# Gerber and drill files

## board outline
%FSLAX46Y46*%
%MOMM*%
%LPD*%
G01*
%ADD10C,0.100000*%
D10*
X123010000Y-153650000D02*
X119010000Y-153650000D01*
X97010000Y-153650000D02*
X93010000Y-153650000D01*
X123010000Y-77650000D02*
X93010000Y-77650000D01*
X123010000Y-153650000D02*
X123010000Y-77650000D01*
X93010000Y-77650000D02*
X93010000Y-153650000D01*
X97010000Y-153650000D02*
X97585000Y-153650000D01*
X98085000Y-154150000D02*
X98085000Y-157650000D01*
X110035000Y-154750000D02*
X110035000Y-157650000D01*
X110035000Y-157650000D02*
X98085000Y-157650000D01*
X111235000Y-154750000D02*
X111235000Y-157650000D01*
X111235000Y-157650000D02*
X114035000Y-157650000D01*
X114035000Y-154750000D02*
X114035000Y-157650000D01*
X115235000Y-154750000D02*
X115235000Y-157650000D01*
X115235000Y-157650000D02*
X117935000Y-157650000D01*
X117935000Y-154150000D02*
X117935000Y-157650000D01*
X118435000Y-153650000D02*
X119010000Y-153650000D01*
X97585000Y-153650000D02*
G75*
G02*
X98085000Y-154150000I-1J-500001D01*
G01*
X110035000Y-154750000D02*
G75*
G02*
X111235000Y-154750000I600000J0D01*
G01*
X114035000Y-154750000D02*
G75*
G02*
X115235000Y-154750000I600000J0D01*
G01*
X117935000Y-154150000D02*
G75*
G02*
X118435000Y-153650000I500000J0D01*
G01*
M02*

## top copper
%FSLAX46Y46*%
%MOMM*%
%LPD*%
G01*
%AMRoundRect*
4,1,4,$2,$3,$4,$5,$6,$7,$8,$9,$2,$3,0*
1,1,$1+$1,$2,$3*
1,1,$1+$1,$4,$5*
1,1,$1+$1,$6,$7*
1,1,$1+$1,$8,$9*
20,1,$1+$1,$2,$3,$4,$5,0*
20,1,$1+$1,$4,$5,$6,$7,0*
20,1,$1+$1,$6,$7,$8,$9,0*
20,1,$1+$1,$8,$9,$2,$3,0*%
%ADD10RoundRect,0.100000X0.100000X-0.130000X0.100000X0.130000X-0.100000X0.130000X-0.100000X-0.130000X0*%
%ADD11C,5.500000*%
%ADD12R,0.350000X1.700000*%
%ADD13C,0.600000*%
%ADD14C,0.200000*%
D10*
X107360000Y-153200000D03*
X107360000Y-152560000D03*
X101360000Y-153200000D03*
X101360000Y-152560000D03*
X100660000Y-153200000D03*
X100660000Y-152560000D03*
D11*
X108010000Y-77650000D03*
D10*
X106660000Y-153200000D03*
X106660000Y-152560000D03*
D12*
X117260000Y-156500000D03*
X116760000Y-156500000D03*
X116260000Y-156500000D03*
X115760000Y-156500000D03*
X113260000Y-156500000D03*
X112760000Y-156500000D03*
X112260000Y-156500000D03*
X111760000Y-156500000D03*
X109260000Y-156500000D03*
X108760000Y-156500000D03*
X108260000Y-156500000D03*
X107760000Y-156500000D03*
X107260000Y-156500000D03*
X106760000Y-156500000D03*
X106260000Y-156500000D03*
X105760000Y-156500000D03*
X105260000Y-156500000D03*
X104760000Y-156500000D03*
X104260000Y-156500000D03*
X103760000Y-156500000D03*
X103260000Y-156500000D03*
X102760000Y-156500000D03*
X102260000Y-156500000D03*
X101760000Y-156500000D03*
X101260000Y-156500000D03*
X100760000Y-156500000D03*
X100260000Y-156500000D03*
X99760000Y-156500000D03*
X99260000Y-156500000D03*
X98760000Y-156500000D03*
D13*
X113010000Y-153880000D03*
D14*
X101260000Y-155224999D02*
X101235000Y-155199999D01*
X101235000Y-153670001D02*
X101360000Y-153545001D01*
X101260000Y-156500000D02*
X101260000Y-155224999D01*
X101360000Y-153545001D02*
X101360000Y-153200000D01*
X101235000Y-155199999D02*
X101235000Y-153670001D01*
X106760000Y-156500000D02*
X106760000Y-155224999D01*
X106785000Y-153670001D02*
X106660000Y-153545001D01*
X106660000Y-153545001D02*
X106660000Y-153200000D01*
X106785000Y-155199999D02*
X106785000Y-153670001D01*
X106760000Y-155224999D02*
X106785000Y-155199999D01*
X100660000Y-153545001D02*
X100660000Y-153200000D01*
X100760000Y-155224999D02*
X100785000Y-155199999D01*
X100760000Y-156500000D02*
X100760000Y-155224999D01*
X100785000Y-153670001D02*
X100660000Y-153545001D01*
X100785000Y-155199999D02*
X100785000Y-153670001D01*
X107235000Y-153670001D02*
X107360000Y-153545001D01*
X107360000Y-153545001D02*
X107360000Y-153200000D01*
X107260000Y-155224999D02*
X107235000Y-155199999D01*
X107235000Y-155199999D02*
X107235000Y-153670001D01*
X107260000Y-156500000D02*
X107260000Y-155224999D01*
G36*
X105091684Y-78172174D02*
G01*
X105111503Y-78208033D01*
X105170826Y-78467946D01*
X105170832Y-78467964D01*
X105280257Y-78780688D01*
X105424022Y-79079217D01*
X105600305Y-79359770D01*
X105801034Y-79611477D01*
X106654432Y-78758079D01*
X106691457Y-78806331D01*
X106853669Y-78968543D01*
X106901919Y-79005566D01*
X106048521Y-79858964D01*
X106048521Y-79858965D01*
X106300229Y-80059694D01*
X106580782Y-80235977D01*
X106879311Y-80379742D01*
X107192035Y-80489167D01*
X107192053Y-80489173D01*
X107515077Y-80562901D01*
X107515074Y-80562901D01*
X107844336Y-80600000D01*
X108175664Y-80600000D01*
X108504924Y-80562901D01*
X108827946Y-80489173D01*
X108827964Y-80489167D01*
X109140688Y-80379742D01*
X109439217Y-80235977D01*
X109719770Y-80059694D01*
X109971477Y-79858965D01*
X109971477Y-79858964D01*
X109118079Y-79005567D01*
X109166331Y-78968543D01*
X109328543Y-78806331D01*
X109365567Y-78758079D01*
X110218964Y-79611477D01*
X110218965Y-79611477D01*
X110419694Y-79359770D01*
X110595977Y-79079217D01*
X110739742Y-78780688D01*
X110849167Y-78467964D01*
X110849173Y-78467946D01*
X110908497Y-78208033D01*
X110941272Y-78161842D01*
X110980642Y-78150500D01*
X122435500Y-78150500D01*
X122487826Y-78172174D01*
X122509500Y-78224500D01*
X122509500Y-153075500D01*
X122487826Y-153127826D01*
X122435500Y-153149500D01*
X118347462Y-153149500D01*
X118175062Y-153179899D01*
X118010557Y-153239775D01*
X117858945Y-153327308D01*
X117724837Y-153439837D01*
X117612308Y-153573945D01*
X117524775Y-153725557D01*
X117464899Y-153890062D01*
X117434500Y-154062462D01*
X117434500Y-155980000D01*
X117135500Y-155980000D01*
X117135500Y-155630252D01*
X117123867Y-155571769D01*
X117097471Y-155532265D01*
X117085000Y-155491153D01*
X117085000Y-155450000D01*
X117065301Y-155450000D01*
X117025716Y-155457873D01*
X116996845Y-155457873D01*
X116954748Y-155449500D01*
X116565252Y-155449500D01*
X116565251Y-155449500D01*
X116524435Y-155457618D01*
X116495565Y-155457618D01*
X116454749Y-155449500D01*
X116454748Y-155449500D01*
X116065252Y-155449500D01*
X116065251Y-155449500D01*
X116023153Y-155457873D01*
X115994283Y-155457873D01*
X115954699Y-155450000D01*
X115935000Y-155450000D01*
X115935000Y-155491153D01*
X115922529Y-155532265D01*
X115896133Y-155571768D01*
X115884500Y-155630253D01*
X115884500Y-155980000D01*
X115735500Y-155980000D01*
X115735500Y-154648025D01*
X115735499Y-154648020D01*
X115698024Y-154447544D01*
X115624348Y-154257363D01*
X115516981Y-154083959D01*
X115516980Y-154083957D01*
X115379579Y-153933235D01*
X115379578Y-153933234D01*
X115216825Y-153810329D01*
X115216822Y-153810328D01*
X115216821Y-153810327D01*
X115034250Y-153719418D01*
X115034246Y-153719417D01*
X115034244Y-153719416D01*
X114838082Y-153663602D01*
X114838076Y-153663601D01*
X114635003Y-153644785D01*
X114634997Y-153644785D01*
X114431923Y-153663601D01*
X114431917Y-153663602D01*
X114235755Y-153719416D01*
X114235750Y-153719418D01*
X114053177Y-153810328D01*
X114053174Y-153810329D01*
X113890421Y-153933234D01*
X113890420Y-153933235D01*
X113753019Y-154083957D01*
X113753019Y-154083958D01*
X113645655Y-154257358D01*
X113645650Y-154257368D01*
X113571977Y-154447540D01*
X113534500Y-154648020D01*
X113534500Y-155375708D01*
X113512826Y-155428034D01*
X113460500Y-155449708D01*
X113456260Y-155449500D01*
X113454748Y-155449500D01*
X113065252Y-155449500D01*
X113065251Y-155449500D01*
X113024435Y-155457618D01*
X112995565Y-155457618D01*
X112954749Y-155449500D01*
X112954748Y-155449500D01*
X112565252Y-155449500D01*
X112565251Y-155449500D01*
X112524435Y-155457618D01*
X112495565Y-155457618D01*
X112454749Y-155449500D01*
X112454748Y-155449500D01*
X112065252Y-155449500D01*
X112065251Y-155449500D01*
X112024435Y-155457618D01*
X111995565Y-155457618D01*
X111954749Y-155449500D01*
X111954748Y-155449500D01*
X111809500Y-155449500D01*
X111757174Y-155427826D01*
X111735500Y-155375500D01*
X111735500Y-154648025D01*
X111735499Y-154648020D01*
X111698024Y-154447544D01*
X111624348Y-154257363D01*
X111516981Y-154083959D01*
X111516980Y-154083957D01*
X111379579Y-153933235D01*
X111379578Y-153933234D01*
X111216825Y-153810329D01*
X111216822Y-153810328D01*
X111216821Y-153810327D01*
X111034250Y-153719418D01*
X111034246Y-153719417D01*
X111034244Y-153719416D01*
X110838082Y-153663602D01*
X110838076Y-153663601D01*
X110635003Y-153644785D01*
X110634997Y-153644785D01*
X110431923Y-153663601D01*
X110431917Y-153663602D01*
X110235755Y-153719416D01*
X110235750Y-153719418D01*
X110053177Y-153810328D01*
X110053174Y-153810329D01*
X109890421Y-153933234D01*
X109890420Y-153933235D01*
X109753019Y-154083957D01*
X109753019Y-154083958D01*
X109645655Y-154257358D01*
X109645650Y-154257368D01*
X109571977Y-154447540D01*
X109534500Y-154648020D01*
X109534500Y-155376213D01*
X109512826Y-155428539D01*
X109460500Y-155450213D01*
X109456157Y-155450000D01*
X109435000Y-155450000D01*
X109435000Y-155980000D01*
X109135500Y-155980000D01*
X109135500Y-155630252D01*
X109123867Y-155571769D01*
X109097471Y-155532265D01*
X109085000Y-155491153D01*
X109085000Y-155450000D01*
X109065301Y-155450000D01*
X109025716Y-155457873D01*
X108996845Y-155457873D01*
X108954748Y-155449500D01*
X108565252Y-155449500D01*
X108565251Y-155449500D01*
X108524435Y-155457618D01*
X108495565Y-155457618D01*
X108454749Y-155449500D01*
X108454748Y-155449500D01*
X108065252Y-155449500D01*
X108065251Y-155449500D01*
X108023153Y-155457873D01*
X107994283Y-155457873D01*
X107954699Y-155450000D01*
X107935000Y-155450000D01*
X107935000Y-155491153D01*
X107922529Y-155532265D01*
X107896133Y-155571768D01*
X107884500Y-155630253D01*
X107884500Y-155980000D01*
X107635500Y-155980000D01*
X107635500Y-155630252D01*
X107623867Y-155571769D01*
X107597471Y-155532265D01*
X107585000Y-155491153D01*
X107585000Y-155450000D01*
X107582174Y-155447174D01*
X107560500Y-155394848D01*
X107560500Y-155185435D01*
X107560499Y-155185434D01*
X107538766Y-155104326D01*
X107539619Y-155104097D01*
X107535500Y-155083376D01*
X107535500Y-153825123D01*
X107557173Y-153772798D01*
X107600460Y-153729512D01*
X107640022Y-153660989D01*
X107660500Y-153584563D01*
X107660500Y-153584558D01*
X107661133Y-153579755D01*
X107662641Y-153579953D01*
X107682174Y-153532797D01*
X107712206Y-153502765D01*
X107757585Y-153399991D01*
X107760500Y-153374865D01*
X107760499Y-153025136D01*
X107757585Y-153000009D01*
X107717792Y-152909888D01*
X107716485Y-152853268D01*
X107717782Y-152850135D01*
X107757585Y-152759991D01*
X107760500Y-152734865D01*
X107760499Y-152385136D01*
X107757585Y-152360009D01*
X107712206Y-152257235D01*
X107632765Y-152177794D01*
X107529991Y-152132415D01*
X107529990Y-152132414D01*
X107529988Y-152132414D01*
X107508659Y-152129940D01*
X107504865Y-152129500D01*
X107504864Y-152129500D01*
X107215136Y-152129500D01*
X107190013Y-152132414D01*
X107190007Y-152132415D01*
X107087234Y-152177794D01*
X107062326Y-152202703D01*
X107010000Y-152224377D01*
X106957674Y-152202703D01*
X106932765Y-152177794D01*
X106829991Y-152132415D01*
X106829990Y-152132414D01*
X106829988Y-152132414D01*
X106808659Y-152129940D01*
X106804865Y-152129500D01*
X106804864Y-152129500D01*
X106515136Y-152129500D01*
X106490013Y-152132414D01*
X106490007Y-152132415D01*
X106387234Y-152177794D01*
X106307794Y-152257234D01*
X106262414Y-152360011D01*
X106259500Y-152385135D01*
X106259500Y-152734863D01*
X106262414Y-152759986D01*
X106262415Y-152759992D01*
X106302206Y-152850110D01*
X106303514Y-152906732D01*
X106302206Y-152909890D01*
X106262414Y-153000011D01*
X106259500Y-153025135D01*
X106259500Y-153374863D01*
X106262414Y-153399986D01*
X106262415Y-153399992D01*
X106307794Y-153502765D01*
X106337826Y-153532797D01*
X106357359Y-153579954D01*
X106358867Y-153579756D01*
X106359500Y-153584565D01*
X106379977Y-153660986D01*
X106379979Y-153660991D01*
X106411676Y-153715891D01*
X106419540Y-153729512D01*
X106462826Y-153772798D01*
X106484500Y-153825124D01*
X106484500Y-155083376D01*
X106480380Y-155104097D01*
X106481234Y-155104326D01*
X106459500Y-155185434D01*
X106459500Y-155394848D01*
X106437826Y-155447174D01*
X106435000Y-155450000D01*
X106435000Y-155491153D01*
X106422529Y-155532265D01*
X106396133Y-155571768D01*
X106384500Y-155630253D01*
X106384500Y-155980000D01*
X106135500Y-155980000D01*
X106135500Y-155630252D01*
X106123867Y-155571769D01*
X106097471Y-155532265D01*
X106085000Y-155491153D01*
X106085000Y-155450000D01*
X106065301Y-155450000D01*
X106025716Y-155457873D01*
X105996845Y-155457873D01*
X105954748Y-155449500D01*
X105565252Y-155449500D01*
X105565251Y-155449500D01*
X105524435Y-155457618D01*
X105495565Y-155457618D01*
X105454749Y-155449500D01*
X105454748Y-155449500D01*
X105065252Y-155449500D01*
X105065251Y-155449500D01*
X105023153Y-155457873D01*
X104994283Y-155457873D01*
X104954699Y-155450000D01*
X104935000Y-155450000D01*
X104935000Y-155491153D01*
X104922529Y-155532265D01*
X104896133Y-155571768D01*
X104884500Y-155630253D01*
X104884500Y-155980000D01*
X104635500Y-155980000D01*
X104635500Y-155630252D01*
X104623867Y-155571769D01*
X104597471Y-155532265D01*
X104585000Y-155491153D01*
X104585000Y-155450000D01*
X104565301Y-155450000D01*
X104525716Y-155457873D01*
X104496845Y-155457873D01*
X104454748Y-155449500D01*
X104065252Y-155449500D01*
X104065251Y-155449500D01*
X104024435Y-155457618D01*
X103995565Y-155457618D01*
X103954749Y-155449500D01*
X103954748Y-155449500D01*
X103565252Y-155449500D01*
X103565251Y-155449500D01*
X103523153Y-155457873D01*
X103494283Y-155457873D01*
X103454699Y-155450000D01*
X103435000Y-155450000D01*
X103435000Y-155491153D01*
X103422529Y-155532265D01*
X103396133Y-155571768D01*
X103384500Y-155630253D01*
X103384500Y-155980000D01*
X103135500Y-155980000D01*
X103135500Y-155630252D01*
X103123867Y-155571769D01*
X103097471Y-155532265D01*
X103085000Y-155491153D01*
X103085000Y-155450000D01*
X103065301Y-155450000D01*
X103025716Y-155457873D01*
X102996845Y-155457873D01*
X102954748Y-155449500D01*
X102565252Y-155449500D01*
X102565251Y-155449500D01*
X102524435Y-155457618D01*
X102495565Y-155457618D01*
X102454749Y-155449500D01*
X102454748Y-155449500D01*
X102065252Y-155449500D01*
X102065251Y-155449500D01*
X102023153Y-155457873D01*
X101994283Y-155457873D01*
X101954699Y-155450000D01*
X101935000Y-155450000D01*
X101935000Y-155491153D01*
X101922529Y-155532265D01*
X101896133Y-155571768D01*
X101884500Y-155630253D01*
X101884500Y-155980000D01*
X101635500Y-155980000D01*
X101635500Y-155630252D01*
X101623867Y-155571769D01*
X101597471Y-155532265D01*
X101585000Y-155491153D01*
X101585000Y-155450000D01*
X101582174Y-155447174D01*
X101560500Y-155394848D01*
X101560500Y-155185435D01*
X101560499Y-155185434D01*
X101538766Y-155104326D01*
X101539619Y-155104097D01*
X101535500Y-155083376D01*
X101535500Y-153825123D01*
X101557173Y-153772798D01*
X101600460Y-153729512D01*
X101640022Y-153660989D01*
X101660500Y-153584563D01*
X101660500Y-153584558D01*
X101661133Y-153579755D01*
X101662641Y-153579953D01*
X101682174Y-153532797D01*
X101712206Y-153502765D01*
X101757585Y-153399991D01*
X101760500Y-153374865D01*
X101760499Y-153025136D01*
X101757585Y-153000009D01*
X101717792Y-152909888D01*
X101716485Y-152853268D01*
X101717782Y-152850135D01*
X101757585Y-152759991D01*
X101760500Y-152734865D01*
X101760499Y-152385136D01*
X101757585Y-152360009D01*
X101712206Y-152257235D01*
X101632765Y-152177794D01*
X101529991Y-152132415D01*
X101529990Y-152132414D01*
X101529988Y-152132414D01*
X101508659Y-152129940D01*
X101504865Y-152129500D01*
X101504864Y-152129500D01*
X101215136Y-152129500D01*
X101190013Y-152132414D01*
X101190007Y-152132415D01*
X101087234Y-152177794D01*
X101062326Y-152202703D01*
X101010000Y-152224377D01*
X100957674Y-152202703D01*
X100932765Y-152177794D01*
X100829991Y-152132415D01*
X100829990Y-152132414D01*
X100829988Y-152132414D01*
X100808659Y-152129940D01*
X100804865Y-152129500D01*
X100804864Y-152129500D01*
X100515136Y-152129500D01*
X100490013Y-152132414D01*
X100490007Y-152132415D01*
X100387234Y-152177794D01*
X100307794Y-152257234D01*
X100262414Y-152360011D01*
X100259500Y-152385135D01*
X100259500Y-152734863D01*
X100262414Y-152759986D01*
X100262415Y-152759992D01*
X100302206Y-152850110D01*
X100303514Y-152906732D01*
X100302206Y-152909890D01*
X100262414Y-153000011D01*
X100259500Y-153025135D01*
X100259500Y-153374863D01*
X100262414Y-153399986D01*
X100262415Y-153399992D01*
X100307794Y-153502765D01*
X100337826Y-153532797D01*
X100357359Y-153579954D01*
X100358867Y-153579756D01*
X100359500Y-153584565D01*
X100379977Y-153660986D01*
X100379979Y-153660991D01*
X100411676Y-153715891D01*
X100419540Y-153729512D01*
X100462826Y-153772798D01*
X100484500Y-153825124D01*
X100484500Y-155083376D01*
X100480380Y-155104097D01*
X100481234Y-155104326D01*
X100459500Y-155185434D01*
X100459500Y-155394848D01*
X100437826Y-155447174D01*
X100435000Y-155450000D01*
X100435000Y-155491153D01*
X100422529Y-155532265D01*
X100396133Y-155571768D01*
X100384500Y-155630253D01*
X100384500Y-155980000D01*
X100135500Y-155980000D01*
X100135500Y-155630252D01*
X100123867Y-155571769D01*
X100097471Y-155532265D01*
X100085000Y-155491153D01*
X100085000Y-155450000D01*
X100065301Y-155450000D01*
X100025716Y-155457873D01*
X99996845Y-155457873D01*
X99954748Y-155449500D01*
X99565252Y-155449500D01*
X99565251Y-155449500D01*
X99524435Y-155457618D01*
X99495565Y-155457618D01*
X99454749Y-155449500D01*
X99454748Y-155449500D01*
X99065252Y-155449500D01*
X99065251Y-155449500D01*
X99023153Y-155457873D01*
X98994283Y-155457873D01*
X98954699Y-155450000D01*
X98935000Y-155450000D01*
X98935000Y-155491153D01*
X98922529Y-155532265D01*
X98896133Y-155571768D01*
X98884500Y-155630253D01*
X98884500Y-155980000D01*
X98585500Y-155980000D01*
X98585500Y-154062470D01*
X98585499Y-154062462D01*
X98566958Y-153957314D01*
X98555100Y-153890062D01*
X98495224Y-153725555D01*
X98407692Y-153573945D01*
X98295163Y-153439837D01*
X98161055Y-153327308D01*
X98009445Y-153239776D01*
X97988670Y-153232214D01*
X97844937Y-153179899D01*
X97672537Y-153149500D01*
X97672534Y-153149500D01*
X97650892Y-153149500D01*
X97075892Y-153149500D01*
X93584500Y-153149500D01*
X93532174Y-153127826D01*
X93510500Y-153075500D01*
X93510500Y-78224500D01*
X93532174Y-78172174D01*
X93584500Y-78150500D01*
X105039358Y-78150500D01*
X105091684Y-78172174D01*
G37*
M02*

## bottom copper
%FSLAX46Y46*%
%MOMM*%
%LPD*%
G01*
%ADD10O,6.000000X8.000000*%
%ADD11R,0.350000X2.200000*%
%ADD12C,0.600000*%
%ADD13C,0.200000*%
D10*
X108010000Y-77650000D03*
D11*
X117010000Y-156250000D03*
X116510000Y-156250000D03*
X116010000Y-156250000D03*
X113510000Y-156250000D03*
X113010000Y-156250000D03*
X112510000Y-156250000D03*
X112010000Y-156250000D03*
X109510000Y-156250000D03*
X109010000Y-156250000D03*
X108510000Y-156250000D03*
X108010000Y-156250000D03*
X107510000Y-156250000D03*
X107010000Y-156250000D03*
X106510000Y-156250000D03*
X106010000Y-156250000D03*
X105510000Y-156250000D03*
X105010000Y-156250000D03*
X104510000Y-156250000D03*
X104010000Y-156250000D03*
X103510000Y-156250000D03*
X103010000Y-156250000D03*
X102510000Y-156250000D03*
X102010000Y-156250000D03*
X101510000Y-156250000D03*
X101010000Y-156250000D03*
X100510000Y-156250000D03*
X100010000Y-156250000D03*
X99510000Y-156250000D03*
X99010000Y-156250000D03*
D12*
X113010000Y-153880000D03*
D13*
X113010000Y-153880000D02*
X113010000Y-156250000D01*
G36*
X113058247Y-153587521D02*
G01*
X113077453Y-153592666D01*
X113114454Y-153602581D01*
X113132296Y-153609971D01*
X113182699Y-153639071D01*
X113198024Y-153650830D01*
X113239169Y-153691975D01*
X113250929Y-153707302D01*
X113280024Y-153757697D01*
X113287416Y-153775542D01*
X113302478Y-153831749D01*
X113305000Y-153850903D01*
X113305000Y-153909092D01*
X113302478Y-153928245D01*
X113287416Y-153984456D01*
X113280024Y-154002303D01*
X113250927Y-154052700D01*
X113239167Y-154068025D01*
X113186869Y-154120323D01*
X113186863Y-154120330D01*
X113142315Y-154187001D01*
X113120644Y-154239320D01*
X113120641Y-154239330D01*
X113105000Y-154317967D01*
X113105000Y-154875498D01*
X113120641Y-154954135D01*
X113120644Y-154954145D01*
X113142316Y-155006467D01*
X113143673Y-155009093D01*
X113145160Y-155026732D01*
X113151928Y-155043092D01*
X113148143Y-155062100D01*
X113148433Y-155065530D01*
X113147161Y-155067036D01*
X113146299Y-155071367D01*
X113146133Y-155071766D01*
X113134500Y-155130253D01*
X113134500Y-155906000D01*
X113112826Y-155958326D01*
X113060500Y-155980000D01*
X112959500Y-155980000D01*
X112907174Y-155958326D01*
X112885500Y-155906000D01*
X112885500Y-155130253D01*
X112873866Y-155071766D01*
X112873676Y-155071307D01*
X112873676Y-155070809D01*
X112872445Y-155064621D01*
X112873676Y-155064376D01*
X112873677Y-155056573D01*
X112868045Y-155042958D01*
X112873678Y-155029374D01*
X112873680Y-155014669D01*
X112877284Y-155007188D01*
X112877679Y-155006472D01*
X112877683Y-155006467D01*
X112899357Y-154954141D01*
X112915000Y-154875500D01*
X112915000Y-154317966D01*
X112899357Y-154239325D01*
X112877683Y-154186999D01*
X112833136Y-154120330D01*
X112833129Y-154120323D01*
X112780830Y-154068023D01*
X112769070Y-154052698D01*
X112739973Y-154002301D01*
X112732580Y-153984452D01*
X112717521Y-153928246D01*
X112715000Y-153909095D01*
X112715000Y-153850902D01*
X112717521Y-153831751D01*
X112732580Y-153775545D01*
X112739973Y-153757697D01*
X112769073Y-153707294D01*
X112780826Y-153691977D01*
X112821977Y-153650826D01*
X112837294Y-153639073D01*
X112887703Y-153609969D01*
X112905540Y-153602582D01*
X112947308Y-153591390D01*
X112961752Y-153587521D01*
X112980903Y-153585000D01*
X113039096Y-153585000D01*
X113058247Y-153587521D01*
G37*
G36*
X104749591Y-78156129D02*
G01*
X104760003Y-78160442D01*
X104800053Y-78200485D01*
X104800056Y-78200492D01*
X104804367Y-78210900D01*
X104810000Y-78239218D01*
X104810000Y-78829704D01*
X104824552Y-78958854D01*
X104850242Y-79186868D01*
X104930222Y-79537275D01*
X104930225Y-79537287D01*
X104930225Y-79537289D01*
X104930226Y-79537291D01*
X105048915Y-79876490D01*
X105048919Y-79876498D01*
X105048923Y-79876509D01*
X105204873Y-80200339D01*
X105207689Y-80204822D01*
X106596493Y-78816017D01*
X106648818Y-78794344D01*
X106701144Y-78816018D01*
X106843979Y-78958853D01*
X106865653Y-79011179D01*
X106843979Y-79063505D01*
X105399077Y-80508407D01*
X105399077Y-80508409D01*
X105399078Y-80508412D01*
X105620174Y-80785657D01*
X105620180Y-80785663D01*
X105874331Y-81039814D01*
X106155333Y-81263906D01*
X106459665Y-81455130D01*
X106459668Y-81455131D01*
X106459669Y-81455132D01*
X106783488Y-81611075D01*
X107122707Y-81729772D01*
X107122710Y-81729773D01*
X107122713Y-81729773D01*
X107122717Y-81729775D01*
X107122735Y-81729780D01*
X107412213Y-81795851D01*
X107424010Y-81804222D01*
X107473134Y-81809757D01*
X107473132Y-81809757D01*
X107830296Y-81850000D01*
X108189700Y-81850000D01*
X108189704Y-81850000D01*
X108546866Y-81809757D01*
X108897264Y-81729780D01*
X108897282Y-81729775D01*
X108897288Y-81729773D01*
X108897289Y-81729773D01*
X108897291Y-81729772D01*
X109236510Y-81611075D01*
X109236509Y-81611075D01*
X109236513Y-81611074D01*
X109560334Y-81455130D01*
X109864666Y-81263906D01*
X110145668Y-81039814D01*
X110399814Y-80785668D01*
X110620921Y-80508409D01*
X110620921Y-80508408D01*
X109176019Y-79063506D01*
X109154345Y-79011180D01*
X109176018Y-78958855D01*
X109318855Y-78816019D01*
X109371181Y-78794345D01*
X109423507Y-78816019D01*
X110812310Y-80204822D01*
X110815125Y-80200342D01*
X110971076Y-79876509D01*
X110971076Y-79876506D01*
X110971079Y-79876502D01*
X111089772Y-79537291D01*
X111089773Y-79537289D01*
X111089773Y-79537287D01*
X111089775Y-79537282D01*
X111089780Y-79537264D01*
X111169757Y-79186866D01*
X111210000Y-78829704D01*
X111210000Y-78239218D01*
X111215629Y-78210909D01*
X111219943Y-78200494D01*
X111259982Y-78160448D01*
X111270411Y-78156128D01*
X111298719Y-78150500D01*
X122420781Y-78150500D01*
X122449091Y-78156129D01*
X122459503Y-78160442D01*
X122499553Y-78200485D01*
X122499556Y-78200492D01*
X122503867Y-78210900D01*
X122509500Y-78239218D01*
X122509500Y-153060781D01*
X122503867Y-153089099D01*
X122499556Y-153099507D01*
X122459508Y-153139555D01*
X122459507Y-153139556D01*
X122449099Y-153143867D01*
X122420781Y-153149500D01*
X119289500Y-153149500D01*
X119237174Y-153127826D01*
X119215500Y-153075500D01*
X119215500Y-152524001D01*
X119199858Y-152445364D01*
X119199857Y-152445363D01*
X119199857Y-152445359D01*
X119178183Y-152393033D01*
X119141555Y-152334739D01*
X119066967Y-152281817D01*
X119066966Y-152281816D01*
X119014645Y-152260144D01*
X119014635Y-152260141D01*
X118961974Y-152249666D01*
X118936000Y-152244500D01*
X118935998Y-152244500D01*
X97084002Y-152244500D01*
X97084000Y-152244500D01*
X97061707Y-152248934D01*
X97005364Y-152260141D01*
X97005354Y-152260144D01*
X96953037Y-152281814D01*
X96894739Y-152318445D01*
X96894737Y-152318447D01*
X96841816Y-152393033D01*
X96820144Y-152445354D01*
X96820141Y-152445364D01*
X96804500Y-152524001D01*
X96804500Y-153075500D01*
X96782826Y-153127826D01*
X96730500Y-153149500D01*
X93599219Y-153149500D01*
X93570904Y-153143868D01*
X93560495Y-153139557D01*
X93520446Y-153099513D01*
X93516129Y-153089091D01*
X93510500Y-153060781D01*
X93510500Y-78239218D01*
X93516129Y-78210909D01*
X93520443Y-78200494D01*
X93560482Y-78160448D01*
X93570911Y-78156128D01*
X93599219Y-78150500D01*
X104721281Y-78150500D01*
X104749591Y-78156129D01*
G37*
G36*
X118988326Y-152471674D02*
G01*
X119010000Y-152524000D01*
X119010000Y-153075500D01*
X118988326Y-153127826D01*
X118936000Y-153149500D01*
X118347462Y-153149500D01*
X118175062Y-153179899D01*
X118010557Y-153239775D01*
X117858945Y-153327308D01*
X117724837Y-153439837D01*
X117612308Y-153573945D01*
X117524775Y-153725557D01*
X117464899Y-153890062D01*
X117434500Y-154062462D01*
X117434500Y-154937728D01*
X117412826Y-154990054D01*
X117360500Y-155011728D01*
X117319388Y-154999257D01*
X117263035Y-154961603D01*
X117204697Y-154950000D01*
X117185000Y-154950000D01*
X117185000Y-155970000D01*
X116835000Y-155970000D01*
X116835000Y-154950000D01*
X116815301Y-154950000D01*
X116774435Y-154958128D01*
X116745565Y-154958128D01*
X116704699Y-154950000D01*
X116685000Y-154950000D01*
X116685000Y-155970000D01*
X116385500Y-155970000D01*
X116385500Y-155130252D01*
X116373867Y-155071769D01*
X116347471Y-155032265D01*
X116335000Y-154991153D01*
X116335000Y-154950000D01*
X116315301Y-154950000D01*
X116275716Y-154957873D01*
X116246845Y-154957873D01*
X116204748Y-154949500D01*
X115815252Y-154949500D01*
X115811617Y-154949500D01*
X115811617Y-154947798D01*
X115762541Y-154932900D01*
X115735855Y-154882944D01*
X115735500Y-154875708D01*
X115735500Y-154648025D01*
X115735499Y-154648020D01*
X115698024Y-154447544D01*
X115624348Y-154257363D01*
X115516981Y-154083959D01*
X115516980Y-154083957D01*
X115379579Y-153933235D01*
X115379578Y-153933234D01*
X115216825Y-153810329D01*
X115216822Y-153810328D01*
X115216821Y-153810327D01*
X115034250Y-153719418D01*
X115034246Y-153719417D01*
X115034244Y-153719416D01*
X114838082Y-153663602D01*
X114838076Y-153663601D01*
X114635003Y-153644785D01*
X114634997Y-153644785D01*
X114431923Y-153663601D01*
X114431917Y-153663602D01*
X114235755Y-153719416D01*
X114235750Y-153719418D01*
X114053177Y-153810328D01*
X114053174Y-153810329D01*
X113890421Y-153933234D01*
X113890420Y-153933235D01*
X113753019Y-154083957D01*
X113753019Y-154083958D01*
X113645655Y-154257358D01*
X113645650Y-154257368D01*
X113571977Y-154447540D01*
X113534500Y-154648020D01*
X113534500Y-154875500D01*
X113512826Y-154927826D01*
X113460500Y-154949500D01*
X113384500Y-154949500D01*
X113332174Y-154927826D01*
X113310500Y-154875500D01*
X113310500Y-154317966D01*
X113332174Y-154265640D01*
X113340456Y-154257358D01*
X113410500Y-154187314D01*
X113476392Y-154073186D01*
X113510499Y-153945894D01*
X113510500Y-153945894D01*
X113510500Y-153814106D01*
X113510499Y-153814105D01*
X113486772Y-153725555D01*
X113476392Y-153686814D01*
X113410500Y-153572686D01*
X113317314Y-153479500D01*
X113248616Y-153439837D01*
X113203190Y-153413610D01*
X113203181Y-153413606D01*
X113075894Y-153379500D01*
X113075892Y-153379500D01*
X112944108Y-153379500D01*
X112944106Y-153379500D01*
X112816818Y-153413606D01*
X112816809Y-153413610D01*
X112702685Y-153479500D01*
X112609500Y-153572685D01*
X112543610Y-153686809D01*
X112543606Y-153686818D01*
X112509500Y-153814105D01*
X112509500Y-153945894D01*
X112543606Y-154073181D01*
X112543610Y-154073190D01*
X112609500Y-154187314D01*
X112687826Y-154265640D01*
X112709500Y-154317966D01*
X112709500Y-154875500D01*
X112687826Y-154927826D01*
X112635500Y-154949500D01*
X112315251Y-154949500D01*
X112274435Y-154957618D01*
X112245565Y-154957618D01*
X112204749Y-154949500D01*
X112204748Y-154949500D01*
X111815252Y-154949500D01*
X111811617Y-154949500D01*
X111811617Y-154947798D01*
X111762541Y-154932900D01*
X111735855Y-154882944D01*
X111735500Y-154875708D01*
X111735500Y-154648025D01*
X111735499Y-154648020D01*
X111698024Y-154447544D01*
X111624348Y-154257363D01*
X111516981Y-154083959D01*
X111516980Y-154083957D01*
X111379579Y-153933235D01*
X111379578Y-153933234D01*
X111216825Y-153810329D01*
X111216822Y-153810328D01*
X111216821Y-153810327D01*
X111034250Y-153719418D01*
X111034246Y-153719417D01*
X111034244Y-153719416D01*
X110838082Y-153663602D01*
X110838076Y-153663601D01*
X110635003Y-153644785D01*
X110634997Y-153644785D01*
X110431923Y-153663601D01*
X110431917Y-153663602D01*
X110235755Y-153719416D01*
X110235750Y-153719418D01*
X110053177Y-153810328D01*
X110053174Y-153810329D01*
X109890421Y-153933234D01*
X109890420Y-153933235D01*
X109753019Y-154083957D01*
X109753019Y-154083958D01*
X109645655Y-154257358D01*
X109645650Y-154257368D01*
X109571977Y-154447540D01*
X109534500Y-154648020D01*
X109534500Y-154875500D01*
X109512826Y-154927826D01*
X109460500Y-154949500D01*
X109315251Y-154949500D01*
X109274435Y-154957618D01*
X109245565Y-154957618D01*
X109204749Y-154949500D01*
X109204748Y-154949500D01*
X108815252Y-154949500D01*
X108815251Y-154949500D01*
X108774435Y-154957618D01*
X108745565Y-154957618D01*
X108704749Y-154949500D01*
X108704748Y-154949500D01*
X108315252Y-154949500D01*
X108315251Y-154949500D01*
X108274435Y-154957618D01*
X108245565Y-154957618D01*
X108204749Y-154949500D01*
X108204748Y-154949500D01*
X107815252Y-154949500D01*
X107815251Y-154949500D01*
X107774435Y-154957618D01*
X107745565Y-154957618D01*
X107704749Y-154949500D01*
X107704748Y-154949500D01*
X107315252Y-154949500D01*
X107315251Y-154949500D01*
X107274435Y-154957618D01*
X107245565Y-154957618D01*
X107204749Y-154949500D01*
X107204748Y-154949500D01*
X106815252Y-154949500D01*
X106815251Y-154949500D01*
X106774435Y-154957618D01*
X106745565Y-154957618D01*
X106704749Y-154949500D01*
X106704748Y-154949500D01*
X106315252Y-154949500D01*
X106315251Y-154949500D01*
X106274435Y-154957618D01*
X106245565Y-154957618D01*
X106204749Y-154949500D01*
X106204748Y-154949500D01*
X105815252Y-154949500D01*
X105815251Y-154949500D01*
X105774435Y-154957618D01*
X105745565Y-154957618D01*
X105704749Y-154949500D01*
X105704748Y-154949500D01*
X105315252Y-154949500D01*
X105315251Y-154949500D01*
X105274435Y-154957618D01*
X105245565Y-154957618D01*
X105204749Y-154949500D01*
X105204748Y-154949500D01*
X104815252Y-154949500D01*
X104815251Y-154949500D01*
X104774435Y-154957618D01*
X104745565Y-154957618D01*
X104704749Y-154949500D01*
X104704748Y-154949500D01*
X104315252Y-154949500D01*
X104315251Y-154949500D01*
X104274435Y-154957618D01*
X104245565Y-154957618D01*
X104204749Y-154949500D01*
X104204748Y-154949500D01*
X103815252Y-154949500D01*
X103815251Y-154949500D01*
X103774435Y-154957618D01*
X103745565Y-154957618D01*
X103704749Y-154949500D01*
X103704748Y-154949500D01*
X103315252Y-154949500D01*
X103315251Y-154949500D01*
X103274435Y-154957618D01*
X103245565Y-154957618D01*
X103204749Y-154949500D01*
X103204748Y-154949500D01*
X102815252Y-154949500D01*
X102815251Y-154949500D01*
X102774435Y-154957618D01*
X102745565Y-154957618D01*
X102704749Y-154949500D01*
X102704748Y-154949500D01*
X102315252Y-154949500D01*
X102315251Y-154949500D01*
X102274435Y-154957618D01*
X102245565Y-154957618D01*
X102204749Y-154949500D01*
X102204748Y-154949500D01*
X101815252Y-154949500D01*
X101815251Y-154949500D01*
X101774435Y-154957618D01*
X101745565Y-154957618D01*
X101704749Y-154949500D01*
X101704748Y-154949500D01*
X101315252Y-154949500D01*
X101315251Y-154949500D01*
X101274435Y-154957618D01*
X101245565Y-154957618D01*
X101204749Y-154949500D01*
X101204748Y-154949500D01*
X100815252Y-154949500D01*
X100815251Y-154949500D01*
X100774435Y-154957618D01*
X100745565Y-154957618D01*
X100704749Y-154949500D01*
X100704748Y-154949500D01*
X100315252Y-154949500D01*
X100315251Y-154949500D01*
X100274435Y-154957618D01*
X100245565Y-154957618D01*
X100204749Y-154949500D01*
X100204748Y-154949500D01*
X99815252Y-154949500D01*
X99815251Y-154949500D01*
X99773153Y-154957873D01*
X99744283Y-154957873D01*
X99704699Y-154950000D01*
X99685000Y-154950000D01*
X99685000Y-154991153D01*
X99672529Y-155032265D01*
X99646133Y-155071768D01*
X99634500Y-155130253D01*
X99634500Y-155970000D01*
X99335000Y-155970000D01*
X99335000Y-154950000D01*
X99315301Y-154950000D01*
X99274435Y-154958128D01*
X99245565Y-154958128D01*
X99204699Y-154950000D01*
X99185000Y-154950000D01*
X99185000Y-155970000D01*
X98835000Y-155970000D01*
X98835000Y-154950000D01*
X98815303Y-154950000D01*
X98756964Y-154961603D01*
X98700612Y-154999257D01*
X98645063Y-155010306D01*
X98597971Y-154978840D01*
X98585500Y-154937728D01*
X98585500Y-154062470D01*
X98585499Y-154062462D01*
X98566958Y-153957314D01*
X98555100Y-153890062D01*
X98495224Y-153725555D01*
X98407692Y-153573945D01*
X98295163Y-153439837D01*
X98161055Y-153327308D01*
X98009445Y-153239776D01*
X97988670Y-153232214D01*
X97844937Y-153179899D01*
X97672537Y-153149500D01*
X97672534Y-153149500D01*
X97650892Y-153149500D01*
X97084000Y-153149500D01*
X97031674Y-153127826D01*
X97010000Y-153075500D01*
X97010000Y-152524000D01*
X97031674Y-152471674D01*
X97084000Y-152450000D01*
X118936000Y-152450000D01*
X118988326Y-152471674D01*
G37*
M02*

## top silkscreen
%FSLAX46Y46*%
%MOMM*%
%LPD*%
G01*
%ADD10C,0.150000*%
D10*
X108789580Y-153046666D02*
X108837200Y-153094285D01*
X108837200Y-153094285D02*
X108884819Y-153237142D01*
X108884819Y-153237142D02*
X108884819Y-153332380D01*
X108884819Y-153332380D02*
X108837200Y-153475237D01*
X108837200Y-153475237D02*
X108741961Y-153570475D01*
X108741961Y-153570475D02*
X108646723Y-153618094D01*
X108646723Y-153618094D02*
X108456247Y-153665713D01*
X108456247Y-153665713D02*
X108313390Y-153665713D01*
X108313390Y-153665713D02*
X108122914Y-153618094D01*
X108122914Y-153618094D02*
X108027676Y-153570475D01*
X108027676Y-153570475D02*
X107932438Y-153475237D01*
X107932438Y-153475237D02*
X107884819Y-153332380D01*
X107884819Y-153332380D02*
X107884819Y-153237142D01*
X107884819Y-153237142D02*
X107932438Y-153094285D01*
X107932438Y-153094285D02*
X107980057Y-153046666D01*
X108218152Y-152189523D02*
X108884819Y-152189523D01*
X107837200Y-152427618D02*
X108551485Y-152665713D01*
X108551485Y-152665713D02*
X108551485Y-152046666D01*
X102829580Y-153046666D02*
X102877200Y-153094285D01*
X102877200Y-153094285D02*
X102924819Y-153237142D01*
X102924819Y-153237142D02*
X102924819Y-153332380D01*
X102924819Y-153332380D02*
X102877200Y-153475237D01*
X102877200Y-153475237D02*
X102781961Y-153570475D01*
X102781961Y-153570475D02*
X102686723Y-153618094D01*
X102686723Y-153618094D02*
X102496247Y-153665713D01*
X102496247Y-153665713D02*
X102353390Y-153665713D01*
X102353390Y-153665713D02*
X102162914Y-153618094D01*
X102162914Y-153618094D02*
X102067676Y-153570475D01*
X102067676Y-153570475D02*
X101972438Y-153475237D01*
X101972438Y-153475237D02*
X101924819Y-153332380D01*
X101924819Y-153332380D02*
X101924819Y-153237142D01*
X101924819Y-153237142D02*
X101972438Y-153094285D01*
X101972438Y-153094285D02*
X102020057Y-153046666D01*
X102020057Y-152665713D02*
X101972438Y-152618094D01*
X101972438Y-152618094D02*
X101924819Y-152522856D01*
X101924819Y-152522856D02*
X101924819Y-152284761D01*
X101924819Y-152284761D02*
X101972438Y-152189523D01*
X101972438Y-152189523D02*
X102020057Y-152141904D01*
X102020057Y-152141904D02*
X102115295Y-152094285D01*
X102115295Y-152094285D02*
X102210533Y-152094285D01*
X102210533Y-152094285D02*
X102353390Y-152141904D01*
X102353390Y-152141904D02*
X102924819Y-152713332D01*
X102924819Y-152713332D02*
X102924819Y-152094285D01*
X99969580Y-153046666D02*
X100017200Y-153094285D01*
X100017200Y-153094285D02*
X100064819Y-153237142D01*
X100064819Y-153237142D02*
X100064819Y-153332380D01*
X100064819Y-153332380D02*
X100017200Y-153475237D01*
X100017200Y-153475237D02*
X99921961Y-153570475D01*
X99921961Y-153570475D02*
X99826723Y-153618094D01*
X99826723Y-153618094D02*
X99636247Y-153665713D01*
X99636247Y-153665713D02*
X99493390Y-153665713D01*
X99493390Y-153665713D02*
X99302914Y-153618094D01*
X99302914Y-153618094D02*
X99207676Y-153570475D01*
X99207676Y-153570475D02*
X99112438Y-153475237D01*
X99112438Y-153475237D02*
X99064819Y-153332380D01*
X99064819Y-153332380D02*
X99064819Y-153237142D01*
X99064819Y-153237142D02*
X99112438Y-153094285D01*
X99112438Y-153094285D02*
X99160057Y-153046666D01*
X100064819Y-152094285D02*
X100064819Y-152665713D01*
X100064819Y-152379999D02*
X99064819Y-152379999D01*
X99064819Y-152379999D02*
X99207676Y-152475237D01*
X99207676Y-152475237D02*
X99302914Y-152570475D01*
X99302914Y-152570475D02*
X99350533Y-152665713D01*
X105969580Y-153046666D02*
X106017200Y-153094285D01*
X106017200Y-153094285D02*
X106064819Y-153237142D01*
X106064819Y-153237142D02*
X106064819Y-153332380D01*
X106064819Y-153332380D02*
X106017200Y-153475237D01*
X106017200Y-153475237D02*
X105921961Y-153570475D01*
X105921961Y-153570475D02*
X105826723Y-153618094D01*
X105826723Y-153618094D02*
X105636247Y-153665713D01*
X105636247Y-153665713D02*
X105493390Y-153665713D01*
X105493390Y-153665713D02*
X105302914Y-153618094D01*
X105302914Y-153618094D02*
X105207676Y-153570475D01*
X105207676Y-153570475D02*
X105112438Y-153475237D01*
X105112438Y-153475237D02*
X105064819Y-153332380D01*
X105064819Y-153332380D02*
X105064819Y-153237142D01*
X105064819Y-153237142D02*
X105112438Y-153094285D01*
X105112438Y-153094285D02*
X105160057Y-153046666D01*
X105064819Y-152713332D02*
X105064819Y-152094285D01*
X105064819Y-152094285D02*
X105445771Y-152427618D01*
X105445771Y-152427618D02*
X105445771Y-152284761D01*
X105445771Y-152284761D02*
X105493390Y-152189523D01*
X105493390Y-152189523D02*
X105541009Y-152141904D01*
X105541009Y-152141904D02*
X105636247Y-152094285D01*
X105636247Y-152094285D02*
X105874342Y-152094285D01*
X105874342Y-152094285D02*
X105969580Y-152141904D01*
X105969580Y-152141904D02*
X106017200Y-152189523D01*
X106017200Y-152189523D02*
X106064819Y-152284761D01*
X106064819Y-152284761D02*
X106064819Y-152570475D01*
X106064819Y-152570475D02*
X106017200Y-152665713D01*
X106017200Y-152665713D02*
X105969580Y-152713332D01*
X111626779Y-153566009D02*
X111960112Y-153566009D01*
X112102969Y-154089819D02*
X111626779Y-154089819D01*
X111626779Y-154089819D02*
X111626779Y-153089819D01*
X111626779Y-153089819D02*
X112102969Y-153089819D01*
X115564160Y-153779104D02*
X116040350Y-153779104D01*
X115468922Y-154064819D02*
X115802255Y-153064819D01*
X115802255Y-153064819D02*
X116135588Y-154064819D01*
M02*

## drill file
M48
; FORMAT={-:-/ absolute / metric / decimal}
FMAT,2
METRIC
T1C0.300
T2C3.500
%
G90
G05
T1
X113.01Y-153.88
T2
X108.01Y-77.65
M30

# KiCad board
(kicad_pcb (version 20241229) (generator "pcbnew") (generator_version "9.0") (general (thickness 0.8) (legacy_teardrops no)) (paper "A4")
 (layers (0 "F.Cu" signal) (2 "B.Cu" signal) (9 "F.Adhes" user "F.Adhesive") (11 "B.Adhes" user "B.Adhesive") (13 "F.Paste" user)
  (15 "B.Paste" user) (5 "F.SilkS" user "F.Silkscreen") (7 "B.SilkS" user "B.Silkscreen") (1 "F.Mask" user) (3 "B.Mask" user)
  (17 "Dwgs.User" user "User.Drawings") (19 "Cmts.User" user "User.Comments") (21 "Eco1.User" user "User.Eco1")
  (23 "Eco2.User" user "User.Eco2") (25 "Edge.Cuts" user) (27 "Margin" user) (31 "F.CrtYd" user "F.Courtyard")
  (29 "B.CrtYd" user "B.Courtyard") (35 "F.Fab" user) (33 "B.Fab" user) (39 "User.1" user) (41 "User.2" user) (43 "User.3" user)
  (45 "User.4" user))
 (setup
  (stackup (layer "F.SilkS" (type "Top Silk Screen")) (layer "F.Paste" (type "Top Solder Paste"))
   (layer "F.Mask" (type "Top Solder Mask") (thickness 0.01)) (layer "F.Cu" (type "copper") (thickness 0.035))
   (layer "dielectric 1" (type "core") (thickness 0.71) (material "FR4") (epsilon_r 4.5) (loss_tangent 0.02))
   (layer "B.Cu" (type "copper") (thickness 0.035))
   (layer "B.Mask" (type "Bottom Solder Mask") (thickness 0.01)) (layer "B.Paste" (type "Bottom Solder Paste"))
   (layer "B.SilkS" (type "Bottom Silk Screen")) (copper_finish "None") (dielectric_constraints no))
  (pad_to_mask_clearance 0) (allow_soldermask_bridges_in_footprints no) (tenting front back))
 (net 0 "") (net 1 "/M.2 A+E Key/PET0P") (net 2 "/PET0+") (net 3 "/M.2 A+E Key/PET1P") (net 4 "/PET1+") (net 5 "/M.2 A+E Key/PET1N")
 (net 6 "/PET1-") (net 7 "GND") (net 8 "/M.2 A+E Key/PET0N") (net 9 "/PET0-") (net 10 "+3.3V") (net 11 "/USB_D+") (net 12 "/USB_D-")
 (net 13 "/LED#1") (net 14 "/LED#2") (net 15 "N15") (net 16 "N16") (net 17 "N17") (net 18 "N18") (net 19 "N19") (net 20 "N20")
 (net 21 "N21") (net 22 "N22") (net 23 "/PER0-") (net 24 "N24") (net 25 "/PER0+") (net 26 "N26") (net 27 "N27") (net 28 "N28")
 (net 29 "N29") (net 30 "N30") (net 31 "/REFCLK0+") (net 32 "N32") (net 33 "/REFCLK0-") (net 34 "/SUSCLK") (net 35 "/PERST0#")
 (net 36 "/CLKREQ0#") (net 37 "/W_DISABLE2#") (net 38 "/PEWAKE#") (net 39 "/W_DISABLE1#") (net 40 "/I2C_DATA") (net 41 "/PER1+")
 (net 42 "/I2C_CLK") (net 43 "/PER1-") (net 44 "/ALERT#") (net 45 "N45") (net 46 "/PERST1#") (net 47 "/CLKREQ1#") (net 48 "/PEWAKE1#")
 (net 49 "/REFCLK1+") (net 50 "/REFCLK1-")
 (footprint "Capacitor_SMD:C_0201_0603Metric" (layer "F.Cu") (at 107.36 152.88 90)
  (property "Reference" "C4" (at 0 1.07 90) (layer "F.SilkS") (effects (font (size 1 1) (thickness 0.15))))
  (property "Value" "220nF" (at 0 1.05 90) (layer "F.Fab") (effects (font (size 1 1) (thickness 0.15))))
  (pad "" smd roundrect (at -0.345 0 90) (size 0.318 0.36) (layers "F.Paste") (roundrect_rratio 0.25))
  (pad "" smd roundrect (at 0.345 0 90) (size 0.318 0.36) (layers "F.Paste") (roundrect_rratio 0.25))
  (pad "1" smd roundrect (at -0.32 0 90) (size 0.46 0.4) (layers "F.Cu" "F.Mask") (roundrect_rratio 0.25) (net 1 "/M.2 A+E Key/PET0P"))
  (pad "2" smd roundrect (at 0.32 0 90) (size 0.46 0.4) (layers "F.Cu" "F.Mask") (roundrect_rratio 0.25) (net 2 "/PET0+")))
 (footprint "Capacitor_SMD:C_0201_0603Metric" (layer "F.Cu") (at 101.36 152.88 90)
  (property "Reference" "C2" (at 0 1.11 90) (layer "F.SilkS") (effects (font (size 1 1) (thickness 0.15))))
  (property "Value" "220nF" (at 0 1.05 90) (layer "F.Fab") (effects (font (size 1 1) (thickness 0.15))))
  (pad "" smd roundrect (at -0.345 0 90) (size 0.318 0.36) (layers "F.Paste") (roundrect_rratio 0.25))
  (pad "" smd roundrect (at 0.345 0 90) (size 0.318 0.36) (layers "F.Paste") (roundrect_rratio 0.25))
  (pad "1" smd roundrect (at -0.32 0 90) (size 0.46 0.4) (layers "F.Cu" "F.Mask") (roundrect_rratio 0.25) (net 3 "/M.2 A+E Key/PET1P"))
  (pad "2" smd roundrect (at 0.32 0 90) (size 0.46 0.4) (layers "F.Cu" "F.Mask") (roundrect_rratio 0.25) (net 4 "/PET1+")))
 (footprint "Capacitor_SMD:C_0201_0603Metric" (layer "F.Cu") (at 100.66 152.88 90)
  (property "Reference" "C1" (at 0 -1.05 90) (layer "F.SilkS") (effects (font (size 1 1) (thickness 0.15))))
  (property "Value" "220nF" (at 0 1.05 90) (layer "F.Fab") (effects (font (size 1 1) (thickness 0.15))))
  (pad "" smd roundrect (at -0.345 0 90) (size 0.318 0.36) (layers "F.Paste") (roundrect_rratio 0.25))
  (pad "" smd roundrect (at 0.345 0 90) (size 0.318 0.36) (layers "F.Paste") (roundrect_rratio 0.25))
  (pad "1" smd roundrect (at -0.32 0 90) (size 0.46 0.4) (layers "F.Cu" "F.Mask") (roundrect_rratio 0.25) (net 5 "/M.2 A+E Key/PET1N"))
  (pad "2" smd roundrect (at 0.32 0 90) (size 0.46 0.4) (layers "F.Cu" "F.Mask") (roundrect_rratio 0.25) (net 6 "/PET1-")))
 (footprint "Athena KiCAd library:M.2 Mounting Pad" (layer "F.Cu") (at 108.01 77.65)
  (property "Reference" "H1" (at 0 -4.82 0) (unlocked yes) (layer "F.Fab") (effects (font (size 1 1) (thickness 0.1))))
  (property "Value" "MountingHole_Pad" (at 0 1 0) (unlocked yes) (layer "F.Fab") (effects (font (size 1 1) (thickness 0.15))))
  (pad "1" thru_hole circle (at 0 0) (size 5.5 5.5) (drill 3.5) (layers "*.Cu" "*.Mask") (remove_unused_layers no) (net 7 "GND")
   (padstack (mode front_inner_back)
    (layer "Inner" (shape circle) (size 5.5 5.5) (zone_connect -1))
    (layer "B.Cu" (shape oval) (size 6 8) (thermal_bridge_angle 45) (zone_connect -1)))))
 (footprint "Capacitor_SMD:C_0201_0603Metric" (layer "F.Cu") (at 106.66 152.88 90)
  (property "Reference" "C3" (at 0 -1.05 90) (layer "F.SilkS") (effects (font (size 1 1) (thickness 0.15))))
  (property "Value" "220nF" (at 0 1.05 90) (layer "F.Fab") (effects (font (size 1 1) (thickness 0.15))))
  (pad "" smd roundrect (at -0.345 0 90) (size 0.318 0.36) (layers "F.Paste") (roundrect_rratio 0.25))
  (pad "" smd roundrect (at 0.345 0 90) (size 0.318 0.36) (layers "F.Paste") (roundrect_rratio 0.25))
  (pad "1" smd roundrect (at -0.32 0 90) (size 0.46 0.4) (layers "F.Cu" "F.Mask") (roundrect_rratio 0.25) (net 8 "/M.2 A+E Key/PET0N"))
  (pad "2" smd roundrect (at 0.32 0 90) (size 0.46 0.4) (layers "F.Cu" "F.Mask") (roundrect_rratio 0.25) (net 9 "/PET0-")))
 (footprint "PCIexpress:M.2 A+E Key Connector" (layer "F.Cu") (at 108.01 156.54)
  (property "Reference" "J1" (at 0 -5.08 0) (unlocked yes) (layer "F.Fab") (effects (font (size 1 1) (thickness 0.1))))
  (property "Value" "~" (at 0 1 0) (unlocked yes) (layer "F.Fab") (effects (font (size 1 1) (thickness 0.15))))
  (fp_line (start -11 -2.89) (end -10.425 -2.89) (stroke (width 0.1) (type default)) (layer "Edge.Cuts"))
  (fp_line (start -9.925 -2.39) (end -9.925 1.11) (stroke (width 0.1) (type default)) (layer "Edge.Cuts"))
  (fp_line (start 2.025 -1.79) (end 2.025 1.11) (stroke (width 0.1) (type default)) (layer "Edge.Cuts"))
  (fp_line (start 2.025 1.11) (end -9.925 1.11) (stroke (width 0.1) (type default)) (layer "Edge.Cuts"))
  (fp_line (start 3.225 -1.79) (end 3.225 1.11) (stroke (width 0.1) (type default)) (layer "Edge.Cuts"))
  (fp_line (start 3.225 1.11) (end 6.025 1.11) (stroke (width 0.1) (type default)) (layer "Edge.Cuts"))
  (fp_line (start 6.025 -1.79) (end 6.025 1.11) (stroke (width 0.1) (type default)) (layer "Edge.Cuts"))
  (fp_line (start 7.225 -1.79) (end 7.225 1.11) (stroke (width 0.1) (type default)) (layer "Edge.Cuts"))
  (fp_line (start 7.225 1.11) (end 9.925 1.11) (stroke (width 0.1) (type default)) (layer "Edge.Cuts"))
  (fp_line (start 9.925 -2.39) (end 9.925 1.11) (stroke (width 0.1) (type default)) (layer "Edge.Cuts"))
  (fp_line (start 10.425 -2.89) (end 11 -2.89) (stroke (width 0.1) (type default)) (layer "Edge.Cuts"))
  (fp_arc (start -10.425 -2.89) (mid -10.071447 -2.743553) (end -9.925 -2.39) (stroke (width 0.1) (type default)) (layer "Edge.Cuts"))
  (fp_arc (start 2.025 -1.79) (mid 2.625 -2.39) (end 3.225 -1.79) (stroke (width 0.1) (type default)) (layer "Edge.Cuts"))
  (fp_arc (start 6.025 -1.79) (mid 6.625 -2.39) (end 7.225 -1.79) (stroke (width 0.1) (type default)) (layer "Edge.Cuts"))
  (fp_arc (start 9.925 -2.39) (mid 10.071447 -2.743553) (end 10.425 -2.89) (stroke (width 0.1) (type default)) (layer "Edge.Cuts"))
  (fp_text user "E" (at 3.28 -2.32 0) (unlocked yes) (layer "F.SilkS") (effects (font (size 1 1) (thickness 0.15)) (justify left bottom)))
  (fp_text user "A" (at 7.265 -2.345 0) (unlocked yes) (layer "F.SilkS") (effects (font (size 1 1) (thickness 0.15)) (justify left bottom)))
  (pad "1" smd rect (at 9.25 -0.04 180) (size 0.35 1.7) (layers "F.Cu") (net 7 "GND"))
  (pad "2" smd rect (at 9 -0.29 180) (size 0.35 2.2) (layers "B.Cu") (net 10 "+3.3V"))
  (pad "3" smd rect (at 8.75 -0.04 180) (size 0.35 1.7) (layers "F.Cu") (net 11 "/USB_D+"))
  (pad "4" smd rect (at 8.5 -0.29 180) (size 0.35 2.2) (layers "B.Cu") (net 10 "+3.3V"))
  (pad "5" smd rect (at 8.25 -0.04 180) (size 0.35 1.7) (layers "F.Cu") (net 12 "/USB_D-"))
  (pad "6" smd rect (at 8 -0.29 180) (size 0.35 2.2) (layers "B.Cu") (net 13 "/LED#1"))
  (pad "7" smd rect (at 7.75 -0.04 180) (size 0.35 1.7) (layers "F.Cu") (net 7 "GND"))
  (pad "16" smd rect (at 5.5 -0.29 180) (size 0.35 2.2) (layers "B.Cu") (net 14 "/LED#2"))
  (pad "17" smd rect (at 5.25 -0.04 180) (size 0.35 1.7) (layers "F.Cu") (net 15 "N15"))
  (pad "18" smd rect (at 5 -0.29 180) (size 0.35 2.2) (layers "B.Cu") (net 7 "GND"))
  (pad "19" smd rect (at 4.75 -0.04 180) (size 0.35 1.7) (layers "F.Cu") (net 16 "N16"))
  (pad "20" smd rect (at 4.5 -0.29 180) (size 0.35 2.2) (layers "B.Cu") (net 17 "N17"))
  (pad "21" smd rect (at 4.25 -0.04 180) (size 0.35 1.7) (layers "F.Cu") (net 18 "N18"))
  (pad "22" smd rect (at 4 -0.29 180) (size 0.35 2.2) (layers "B.Cu") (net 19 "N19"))
  (pad "23" smd rect (at 3.75 -0.04 180) (size 0.35 1.7) (layers "F.Cu") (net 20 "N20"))
  (pad "32" smd rect (at 1.5 -0.29 180) (size 0.35 2.2) (layers "B.Cu") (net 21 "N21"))
  (pad "33" smd rect (at 1.25 -0.04 180) (size 0.35 1.7) (layers "F.Cu") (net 7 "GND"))
  (pad "34" smd rect (at 1 -0.29 180) (size 0.35 2.2) (layers "B.Cu") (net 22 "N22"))
  (pad "35" smd rect (at 0.75 -0.04 180) (size 0.35 1.7) (layers "F.Cu") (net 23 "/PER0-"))
  (pad "36" smd rect (at 0.5 -0.29 180) (size 0.35 2.2) (layers "B.Cu") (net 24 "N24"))
  (pad "37" smd rect (at 0.25 -0.04 180) (size 0.35 1.7) (layers "F.Cu") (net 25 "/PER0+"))
  (pad "38" smd rect (at 0 -0.29 180) (size 0.35 2.2) (layers "B.Cu") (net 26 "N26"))
  (pad "39" smd rect (at -0.25 -0.04 180) (size 0.35 1.7) (layers "F.Cu") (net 7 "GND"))
  (pad "40" smd rect (at -0.5 -0.29 180) (size 0.35 2.2) (layers "B.Cu") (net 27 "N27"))
  (pad "41" smd rect (at -0.75 -0.04 180) (size 0.35 1.7) (layers "F.Cu") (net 1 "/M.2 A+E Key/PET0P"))
  (pad "42" smd rect (at -1 -0.29 180) (size 0.35 2.2) (layers "B.Cu") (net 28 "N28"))
  (pad "43" smd rect (at -1.25 -0.04 180) (size 0.35 1.7) (layers "F.Cu") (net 8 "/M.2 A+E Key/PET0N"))
  (pad "44" smd rect (at -1.5 -0.29 180) (size 0.35 2.2) (layers "B.Cu") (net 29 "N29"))
  (pad "45" smd rect (at -1.75 -0.04 180) (size 0.35 1.7) (layers "F.Cu") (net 7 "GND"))
  (pad "46" smd rect (at -2 -0.29 180) (size 0.35 2.2) (layers "B.Cu") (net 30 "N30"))
  (pad "47" smd rect (at -2.25 -0.04 180) (size 0.35 1.7) (layers "F.Cu") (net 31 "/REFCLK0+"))
  (pad "48" smd rect (at -2.5 -0.29 180) (size 0.35 2.2) (layers "B.Cu") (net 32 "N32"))
  (pad "49" smd rect (at -2.75 -0.04 180) (size 0.35 1.7) (layers "F.Cu") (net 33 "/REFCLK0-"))
  (pad "50" smd rect (at -3 -0.29 180) (size 0.35 2.2) (layers "B.Cu") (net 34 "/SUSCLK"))
  (pad "51" smd rect (at -3.25 -0.04 180) (size 0.35 1.7) (layers "F.Cu") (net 7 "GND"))
  (pad "52" smd rect (at -3.5 -0.29 180) (size 0.35 2.2) (layers "B.Cu") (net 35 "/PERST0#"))
  (pad "53" smd rect (at -3.75 -0.04 180) (size 0.35 1.7) (layers "F.Cu") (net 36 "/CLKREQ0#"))
  (pad "54" smd rect (at -4 -0.29 180) (size 0.35 2.2) (layers "B.Cu") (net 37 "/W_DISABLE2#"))
  (pad "55" smd rect (at -4.25 -0.04 180) (size 0.35 1.7) (layers "F.Cu") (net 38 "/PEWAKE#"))
  (pad "56" smd rect (at -4.5 -0.29 180) (size 0.35 2.2) (layers "B.Cu") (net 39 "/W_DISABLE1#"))
  (pad "57" smd rect (at -4.75 -0.04 180) (size 0.35 1.7) (layers "F.Cu") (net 7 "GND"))
  (pad "58" smd rect (at -5 -0.29 180) (size 0.35 2.2) (layers "B.Cu") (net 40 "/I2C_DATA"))
  (pad "59" smd rect (at -5.25 -0.04 180) (size 0.35 1.7) (layers "F.Cu") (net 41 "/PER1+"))
  (pad "60" smd rect (at -5.5 -0.29 180) (size 0.35 2.2) (layers "B.Cu") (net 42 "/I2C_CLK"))
  (pad "61" smd rect (at -5.75 -0.04 180) (size 0.35 1.7) (layers "F.Cu") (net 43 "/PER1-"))
  (pad "62" smd rect (at -6 -0.29 180) (size 0.35 2.2) (layers "B.Cu") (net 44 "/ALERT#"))
  (pad "63" smd rect (at -6.25 -0.04 180) (size 0.35 1.7) (layers "F.Cu") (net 7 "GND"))
  (pad "64" smd rect (at -6.5 -0.29 180) (size 0.35 2.2) (layers "B.Cu") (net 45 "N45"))
  (pad "65" smd rect (at -6.75 -0.04 180) (size 0.35 1.7) (layers "F.Cu") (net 3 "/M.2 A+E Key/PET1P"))
  (pad "66" smd rect (at -7 -0.29 180) (size 0.35 2.2) (layers "B.Cu") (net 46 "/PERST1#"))
  (pad "67" smd rect (at -7.25 -0.04 180) (size 0.35 1.7) (layers "F.Cu") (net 5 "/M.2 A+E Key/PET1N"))
  (pad "68" smd rect (at -7.5 -0.29 180) (size 0.35 2.2) (layers "B.Cu") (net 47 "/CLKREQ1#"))
  (pad "69" smd rect (at -7.75 -0.04 180) (size 0.35 1.7) (layers "F.Cu") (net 7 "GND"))
  (pad "70" smd rect (at -8 -0.29 180) (size 0.35 2.2) (layers "B.Cu") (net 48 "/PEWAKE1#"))
  (pad "71" smd rect (at -8.25 -0.04 180) (size 0.35 1.7) (layers "F.Cu") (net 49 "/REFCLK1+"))
  (pad "72" smd rect (at -8.5 -0.29 180) (size 0.35 2.2) (layers "B.Cu") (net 10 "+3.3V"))
  (pad "73" smd rect (at -8.75 -0.04 180) (size 0.35 1.7) (layers "F.Cu") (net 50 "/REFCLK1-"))
  (pad "74" smd rect (at -9 -0.29 180) (size 0.35 2.2) (layers "B.Cu") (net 10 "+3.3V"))
  (pad "75" smd rect (at -9.25 -0.04 180) (size 0.35 1.7) (layers "F.Cu") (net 7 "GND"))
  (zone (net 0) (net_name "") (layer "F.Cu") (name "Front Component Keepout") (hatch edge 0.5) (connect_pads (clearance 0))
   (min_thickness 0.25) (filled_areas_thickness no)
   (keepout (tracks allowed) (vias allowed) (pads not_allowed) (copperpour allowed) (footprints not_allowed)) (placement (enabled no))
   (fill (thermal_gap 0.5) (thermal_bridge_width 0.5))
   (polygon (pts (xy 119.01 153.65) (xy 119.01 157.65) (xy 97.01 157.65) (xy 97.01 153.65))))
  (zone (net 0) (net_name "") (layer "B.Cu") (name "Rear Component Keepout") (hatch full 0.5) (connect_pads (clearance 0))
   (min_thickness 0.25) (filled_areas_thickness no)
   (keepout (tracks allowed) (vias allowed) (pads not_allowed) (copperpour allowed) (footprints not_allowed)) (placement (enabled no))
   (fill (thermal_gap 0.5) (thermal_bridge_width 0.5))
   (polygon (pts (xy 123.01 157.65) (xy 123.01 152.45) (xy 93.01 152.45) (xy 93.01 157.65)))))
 (gr_line (start 123.01 153.65) (end 119.01 153.65) (stroke (width 0.1) (type default)) (layer "Edge.Cuts"))
 (gr_line (start 97.01 153.65) (end 93.01 153.65) (stroke (width 0.1) (type default)) (layer "Edge.Cuts"))
 (gr_line (start 123.01 77.65) (end 93.01 77.65) (stroke (width 0.1) (type default)) (layer "Edge.Cuts"))
 (gr_line (start 123.01 153.65) (end 123.01 77.65) (stroke (width 0.1) (type default)) (layer "Edge.Cuts"))
 (gr_line (start 93.01 77.65) (end 93.01 153.65) (stroke (width 0.1) (type default)) (layer "Edge.Cuts"))
 (via (at 113.01 153.88) (size 0.6) (drill 0.3) (layers "F.Cu" "B.Cu") (free yes) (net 7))
 (segment (start 113.01 153.88) (end 113.01 156.25) (width 0.2) (layer "B.Cu") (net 7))
 (segment (start 101.26 155.224999) (end 101.235 155.199999) (width 0.2) (layer "F.Cu") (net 3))
 (segment (start 101.235 153.670001) (end 101.36 153.545001) (width 0.2) (layer "F.Cu") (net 3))
 (segment (start 101.26 156.5) (end 101.26 155.224999) (width 0.2) (layer "F.Cu") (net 3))
 (segment (start 101.36 153.545001) (end 101.36 153.2) (width 0.2) (layer "F.Cu") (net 3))
 (segment (start 101.235 155.199999) (end 101.235 153.670001) (width 0.2) (layer "F.Cu") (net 3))
 (segment (start 106.76 156.5) (end 106.76 155.224999) (width 0.2) (layer "F.Cu") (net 8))
 (segment (start 106.785 153.670001) (end 106.66 153.545001) (width 0.2) (layer "F.Cu") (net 8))
 (segment (start 106.66 153.545001) (end 106.66 153.2) (width 0.2) (layer "F.Cu") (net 8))
 (segment (start 106.785 155.199999) (end 106.785 153.670001) (width 0.2) (layer "F.Cu") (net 8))
 (segment (start 106.76 155.224999) (end 106.785 155.199999) (width 0.2) (layer "F.Cu") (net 8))
 (segment (start 100.66 153.545001) (end 100.66 153.2) (width 0.2) (layer "F.Cu") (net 5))
 (segment (start 100.76 155.224999) (end 100.785 155.199999) (width 0.2) (layer "F.Cu") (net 5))
 (segment (start 100.76 156.5) (end 100.76 155.224999) (width 0.2) (layer "F.Cu") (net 5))
 (segment (start 100.785 153.670001) (end 100.66 153.545001) (width 0.2) (layer "F.Cu") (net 5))
 (segment (start 100.785 155.199999) (end 100.785 153.670001) (width 0.2) (layer "F.Cu") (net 5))
 (segment (start 107.235 153.670001) (end 107.36 153.545001) (width 0.2) (layer "F.Cu") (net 1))
 (segment (start 107.36 153.545001) (end 107.36 153.2) (width 0.2) (layer "F.Cu") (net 1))
 (segment (start 107.26 155.224999) (end 107.235 155.199999) (width 0.2) (layer "F.Cu") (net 1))
 (segment (start 107.235 155.199999) (end 107.235 153.670001) (width 0.2) (layer "F.Cu") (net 1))
 (segment (start 107.26 156.5) (end 107.26 155.224999) (width 0.2) (layer "F.Cu") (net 1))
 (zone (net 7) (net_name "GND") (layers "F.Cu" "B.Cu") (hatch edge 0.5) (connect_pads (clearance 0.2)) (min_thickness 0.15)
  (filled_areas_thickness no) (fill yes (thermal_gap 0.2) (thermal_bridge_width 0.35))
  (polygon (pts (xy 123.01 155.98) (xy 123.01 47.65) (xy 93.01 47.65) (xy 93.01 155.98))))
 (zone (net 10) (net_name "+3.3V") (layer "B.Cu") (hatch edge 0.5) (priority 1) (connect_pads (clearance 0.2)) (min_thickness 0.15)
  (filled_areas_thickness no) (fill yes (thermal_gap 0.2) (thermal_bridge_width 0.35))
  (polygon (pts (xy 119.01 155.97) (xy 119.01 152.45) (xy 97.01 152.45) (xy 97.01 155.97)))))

